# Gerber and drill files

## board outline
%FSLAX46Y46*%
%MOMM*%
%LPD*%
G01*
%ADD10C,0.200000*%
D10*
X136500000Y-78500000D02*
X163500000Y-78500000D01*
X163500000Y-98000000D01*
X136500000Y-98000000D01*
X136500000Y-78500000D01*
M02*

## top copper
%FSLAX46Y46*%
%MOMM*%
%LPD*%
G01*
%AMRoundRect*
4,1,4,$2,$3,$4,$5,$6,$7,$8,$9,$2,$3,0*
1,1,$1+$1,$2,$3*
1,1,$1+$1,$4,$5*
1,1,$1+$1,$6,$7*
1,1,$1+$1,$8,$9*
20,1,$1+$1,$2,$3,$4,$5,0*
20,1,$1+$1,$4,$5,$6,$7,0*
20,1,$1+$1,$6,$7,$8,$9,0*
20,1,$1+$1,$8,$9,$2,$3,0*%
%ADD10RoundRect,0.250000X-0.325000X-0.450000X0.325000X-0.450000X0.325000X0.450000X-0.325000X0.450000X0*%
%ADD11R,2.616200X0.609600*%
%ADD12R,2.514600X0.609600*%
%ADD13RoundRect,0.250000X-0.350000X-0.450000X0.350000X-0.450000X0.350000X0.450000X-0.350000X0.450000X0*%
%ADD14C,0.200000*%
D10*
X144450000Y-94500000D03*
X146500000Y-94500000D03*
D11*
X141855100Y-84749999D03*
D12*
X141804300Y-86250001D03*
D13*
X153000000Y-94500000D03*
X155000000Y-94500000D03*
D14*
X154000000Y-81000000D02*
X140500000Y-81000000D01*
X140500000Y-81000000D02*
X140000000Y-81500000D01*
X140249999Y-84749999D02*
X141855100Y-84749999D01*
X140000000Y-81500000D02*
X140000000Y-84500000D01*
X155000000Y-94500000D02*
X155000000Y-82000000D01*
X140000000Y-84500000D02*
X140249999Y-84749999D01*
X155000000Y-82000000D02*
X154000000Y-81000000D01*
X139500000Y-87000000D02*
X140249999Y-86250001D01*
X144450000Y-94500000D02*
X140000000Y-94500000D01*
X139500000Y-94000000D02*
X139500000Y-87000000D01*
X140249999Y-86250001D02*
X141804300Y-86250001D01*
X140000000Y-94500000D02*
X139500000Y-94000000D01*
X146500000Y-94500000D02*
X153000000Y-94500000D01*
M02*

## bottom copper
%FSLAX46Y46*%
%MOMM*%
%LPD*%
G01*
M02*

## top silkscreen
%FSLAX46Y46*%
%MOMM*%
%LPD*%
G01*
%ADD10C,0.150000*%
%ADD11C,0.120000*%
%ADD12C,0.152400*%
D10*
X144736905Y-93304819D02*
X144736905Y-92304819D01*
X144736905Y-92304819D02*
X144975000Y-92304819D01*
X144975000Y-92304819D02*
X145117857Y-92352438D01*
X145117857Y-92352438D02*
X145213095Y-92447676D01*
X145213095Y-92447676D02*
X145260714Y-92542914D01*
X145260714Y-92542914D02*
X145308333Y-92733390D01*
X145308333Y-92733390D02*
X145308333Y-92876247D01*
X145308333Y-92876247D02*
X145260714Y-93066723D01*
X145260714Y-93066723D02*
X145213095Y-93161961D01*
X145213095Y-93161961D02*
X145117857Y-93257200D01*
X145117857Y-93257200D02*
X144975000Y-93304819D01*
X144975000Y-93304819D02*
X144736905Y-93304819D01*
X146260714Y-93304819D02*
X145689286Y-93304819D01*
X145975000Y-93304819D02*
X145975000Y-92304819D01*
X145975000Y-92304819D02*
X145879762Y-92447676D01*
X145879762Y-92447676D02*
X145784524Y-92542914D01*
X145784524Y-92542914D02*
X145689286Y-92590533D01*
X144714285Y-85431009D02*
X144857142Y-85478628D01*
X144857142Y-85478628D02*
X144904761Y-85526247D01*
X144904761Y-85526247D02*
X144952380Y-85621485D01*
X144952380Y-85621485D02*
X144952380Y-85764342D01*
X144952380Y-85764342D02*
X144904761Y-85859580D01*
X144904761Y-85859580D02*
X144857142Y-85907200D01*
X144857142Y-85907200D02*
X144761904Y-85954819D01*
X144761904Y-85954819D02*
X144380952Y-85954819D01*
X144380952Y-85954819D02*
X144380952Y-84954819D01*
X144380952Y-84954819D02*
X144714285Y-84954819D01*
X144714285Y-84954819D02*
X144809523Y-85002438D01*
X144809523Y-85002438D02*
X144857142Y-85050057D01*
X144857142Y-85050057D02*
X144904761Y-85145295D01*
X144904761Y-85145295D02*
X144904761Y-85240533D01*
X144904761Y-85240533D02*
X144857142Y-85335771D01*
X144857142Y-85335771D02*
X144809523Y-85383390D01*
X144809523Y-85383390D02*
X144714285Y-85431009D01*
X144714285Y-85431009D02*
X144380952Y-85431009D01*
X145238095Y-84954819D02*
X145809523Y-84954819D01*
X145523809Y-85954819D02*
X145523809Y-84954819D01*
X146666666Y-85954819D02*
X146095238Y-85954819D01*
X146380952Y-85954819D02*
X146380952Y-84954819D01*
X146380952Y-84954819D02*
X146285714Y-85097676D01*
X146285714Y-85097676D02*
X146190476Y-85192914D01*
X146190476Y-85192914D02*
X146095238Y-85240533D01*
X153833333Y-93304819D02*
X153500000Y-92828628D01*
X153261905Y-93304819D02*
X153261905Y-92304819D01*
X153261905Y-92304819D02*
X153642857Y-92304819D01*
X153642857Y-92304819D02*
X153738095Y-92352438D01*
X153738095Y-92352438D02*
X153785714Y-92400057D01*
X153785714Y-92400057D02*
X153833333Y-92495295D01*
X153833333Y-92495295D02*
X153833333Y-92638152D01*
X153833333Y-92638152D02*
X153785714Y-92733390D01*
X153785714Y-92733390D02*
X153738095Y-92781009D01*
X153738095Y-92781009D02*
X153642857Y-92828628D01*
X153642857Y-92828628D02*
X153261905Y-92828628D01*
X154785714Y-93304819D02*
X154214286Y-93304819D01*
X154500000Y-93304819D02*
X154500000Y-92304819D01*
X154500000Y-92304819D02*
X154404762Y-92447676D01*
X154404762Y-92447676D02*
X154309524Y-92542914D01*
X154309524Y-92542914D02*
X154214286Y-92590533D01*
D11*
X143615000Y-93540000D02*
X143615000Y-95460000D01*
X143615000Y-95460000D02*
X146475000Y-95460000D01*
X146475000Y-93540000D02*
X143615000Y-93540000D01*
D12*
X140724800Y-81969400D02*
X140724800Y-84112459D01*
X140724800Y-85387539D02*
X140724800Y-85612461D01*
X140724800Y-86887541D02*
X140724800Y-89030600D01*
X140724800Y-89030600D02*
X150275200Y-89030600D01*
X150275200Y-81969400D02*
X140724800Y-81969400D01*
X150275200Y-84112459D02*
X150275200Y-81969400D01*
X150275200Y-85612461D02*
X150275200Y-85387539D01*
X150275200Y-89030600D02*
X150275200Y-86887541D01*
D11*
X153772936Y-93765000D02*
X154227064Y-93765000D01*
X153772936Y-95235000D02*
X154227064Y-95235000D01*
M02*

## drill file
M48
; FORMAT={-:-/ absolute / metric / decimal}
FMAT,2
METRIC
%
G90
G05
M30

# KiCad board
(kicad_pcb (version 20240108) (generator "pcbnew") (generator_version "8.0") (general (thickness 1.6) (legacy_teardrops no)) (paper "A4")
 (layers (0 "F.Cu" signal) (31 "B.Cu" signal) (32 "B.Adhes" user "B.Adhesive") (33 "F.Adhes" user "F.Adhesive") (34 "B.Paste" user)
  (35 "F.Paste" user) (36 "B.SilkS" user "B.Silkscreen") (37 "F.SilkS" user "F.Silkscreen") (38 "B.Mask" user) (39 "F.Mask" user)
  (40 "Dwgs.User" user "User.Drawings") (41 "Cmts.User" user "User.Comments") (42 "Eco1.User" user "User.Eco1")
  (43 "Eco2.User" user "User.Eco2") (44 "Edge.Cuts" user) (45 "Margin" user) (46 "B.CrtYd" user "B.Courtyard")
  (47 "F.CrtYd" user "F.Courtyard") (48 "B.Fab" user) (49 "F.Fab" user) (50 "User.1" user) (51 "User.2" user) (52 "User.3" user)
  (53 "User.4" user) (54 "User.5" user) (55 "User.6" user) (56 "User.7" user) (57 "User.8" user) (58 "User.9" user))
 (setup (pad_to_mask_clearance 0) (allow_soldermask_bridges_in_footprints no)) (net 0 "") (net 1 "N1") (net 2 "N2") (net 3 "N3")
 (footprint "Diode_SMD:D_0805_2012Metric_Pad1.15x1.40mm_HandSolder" (layer "F.Cu") (at 145.475 94.5)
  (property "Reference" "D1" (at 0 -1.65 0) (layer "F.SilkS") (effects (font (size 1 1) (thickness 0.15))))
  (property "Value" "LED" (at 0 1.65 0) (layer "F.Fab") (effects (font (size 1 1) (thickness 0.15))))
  (fp_line (start -1.86 -0.96) (end -1.86 0.96) (stroke (width 0.12) (type solid)) (layer "F.SilkS"))
  (fp_line (start -1.86 0.96) (end 1 0.96) (stroke (width 0.12) (type solid)) (layer "F.SilkS"))
  (fp_line (start 1 -0.96) (end -1.86 -0.96) (stroke (width 0.12) (type solid)) (layer "F.SilkS"))
  (pad "1" smd roundrect (at -1.025 0) (size 1.15 1.4) (layers "F.Cu" "F.Paste" "F.Mask") (roundrect_rratio 0.217391) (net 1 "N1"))
  (pad "2" smd roundrect (at 1.025 0) (size 1.15 1.4) (layers "F.Cu" "F.Paste" "F.Mask") (roundrect_rratio 0.217391) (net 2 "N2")))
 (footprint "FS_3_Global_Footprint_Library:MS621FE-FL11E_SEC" (layer "F.Cu") (at 145.5 85.5)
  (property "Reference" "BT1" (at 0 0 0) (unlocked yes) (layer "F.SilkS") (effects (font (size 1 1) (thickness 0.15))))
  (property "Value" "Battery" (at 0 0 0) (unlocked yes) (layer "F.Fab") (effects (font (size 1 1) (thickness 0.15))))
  (fp_line (start -4.7752 -3.5306) (end -4.7752 -1.387541) (stroke (width 0.1524) (type solid)) (layer "F.SilkS"))
  (fp_line (start -4.7752 -0.112461) (end -4.7752 0.112461) (stroke (width 0.1524) (type solid)) (layer "F.SilkS"))
  (fp_line (start -4.7752 1.387541) (end -4.7752 3.5306) (stroke (width 0.1524) (type solid)) (layer "F.SilkS"))
  (fp_line (start -4.7752 3.5306) (end 4.7752 3.5306) (stroke (width 0.1524) (type solid)) (layer "F.SilkS"))
  (fp_line (start 4.7752 -3.5306) (end -4.7752 -3.5306) (stroke (width 0.1524) (type solid)) (layer "F.SilkS"))
  (fp_line (start 4.7752 -1.387541) (end 4.7752 -3.5306) (stroke (width 0.1524) (type solid)) (layer "F.SilkS"))
  (fp_line (start 4.7752 0.112461) (end 4.7752 -0.112461) (stroke (width 0.1524) (type solid)) (layer "F.SilkS"))
  (fp_line (start 4.7752 3.5306) (end 4.7752 1.387541) (stroke (width 0.1524) (type solid)) (layer "F.SilkS"))
  (pad "1" smd rect (at -3.6449 -0.750001) (size 2.6162 0.6096) (layers "F.Cu" "F.Paste" "F.Mask") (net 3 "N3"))
  (pad "2" smd rect (at -3.6957 0.750001) (size 2.5146 0.6096) (layers "F.Cu" "F.Paste" "F.Mask") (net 1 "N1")))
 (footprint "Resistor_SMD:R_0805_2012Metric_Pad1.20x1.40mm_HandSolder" (layer "F.Cu") (at 154 94.5)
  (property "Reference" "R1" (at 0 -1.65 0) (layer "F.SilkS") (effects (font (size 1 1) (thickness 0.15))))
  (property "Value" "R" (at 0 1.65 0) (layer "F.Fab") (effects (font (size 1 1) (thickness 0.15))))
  (fp_line (start -0.227064 -0.735) (end 0.227064 -0.735) (stroke (width 0.12) (type solid)) (layer "F.SilkS"))
  (fp_line (start -0.227064 0.735) (end 0.227064 0.735) (stroke (width 0.12) (type solid)) (layer "F.SilkS"))
  (pad "1" smd roundrect (at -1 0) (size 1.2 1.4) (layers "F.Cu" "F.Paste" "F.Mask") (roundrect_rratio 0.208333) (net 2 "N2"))
  (pad "2" smd roundrect (at 1 0) (size 1.2 1.4) (layers "F.Cu" "F.Paste" "F.Mask") (roundrect_rratio 0.208333) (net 3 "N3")))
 (gr_rect (start 136.5 78.5) (end 163.5 98) (stroke (width 0.2) (type default)) (fill none) (layer "Edge.Cuts"))
 (segment (start 154 81) (end 140.5 81) (width 0.2) (layer "F.Cu") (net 3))
 (segment (start 140.5 81) (end 140 81.5) (width 0.2) (layer "F.Cu") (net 3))
 (segment (start 140.249999 84.749999) (end 141.8551 84.749999) (width 0.2) (layer "F.Cu") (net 3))
 (segment (start 140 81.5) (end 140 84.5) (width 0.2) (layer "F.Cu") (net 3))
 (segment (start 155 94.5) (end 155 82) (width 0.2) (layer "F.Cu") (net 3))
 (segment (start 140 84.5) (end 140.249999 84.749999) (width 0.2) (layer "F.Cu") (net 3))
 (segment (start 155 82) (end 154 81) (width 0.2) (layer "F.Cu") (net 3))
 (segment (start 139.5 87) (end 140.249999 86.250001) (width 0.2) (layer "F.Cu") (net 1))
 (segment (start 144.45 94.5) (end 140 94.5) (width 0.2) (layer "F.Cu") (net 1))
 (segment (start 139.5 94) (end 139.5 87) (width 0.2) (layer "F.Cu") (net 1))
 (segment (start 140.249999 86.250001) (end 141.8043 86.250001) (width 0.2) (layer "F.Cu") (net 1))
 (segment (start 140 94.5) (end 139.5 94) (width 0.2) (layer "F.Cu") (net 1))
 (segment (start 146.5 94.5) (end 153 94.5) (width 0.2) (layer "F.Cu") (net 2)))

